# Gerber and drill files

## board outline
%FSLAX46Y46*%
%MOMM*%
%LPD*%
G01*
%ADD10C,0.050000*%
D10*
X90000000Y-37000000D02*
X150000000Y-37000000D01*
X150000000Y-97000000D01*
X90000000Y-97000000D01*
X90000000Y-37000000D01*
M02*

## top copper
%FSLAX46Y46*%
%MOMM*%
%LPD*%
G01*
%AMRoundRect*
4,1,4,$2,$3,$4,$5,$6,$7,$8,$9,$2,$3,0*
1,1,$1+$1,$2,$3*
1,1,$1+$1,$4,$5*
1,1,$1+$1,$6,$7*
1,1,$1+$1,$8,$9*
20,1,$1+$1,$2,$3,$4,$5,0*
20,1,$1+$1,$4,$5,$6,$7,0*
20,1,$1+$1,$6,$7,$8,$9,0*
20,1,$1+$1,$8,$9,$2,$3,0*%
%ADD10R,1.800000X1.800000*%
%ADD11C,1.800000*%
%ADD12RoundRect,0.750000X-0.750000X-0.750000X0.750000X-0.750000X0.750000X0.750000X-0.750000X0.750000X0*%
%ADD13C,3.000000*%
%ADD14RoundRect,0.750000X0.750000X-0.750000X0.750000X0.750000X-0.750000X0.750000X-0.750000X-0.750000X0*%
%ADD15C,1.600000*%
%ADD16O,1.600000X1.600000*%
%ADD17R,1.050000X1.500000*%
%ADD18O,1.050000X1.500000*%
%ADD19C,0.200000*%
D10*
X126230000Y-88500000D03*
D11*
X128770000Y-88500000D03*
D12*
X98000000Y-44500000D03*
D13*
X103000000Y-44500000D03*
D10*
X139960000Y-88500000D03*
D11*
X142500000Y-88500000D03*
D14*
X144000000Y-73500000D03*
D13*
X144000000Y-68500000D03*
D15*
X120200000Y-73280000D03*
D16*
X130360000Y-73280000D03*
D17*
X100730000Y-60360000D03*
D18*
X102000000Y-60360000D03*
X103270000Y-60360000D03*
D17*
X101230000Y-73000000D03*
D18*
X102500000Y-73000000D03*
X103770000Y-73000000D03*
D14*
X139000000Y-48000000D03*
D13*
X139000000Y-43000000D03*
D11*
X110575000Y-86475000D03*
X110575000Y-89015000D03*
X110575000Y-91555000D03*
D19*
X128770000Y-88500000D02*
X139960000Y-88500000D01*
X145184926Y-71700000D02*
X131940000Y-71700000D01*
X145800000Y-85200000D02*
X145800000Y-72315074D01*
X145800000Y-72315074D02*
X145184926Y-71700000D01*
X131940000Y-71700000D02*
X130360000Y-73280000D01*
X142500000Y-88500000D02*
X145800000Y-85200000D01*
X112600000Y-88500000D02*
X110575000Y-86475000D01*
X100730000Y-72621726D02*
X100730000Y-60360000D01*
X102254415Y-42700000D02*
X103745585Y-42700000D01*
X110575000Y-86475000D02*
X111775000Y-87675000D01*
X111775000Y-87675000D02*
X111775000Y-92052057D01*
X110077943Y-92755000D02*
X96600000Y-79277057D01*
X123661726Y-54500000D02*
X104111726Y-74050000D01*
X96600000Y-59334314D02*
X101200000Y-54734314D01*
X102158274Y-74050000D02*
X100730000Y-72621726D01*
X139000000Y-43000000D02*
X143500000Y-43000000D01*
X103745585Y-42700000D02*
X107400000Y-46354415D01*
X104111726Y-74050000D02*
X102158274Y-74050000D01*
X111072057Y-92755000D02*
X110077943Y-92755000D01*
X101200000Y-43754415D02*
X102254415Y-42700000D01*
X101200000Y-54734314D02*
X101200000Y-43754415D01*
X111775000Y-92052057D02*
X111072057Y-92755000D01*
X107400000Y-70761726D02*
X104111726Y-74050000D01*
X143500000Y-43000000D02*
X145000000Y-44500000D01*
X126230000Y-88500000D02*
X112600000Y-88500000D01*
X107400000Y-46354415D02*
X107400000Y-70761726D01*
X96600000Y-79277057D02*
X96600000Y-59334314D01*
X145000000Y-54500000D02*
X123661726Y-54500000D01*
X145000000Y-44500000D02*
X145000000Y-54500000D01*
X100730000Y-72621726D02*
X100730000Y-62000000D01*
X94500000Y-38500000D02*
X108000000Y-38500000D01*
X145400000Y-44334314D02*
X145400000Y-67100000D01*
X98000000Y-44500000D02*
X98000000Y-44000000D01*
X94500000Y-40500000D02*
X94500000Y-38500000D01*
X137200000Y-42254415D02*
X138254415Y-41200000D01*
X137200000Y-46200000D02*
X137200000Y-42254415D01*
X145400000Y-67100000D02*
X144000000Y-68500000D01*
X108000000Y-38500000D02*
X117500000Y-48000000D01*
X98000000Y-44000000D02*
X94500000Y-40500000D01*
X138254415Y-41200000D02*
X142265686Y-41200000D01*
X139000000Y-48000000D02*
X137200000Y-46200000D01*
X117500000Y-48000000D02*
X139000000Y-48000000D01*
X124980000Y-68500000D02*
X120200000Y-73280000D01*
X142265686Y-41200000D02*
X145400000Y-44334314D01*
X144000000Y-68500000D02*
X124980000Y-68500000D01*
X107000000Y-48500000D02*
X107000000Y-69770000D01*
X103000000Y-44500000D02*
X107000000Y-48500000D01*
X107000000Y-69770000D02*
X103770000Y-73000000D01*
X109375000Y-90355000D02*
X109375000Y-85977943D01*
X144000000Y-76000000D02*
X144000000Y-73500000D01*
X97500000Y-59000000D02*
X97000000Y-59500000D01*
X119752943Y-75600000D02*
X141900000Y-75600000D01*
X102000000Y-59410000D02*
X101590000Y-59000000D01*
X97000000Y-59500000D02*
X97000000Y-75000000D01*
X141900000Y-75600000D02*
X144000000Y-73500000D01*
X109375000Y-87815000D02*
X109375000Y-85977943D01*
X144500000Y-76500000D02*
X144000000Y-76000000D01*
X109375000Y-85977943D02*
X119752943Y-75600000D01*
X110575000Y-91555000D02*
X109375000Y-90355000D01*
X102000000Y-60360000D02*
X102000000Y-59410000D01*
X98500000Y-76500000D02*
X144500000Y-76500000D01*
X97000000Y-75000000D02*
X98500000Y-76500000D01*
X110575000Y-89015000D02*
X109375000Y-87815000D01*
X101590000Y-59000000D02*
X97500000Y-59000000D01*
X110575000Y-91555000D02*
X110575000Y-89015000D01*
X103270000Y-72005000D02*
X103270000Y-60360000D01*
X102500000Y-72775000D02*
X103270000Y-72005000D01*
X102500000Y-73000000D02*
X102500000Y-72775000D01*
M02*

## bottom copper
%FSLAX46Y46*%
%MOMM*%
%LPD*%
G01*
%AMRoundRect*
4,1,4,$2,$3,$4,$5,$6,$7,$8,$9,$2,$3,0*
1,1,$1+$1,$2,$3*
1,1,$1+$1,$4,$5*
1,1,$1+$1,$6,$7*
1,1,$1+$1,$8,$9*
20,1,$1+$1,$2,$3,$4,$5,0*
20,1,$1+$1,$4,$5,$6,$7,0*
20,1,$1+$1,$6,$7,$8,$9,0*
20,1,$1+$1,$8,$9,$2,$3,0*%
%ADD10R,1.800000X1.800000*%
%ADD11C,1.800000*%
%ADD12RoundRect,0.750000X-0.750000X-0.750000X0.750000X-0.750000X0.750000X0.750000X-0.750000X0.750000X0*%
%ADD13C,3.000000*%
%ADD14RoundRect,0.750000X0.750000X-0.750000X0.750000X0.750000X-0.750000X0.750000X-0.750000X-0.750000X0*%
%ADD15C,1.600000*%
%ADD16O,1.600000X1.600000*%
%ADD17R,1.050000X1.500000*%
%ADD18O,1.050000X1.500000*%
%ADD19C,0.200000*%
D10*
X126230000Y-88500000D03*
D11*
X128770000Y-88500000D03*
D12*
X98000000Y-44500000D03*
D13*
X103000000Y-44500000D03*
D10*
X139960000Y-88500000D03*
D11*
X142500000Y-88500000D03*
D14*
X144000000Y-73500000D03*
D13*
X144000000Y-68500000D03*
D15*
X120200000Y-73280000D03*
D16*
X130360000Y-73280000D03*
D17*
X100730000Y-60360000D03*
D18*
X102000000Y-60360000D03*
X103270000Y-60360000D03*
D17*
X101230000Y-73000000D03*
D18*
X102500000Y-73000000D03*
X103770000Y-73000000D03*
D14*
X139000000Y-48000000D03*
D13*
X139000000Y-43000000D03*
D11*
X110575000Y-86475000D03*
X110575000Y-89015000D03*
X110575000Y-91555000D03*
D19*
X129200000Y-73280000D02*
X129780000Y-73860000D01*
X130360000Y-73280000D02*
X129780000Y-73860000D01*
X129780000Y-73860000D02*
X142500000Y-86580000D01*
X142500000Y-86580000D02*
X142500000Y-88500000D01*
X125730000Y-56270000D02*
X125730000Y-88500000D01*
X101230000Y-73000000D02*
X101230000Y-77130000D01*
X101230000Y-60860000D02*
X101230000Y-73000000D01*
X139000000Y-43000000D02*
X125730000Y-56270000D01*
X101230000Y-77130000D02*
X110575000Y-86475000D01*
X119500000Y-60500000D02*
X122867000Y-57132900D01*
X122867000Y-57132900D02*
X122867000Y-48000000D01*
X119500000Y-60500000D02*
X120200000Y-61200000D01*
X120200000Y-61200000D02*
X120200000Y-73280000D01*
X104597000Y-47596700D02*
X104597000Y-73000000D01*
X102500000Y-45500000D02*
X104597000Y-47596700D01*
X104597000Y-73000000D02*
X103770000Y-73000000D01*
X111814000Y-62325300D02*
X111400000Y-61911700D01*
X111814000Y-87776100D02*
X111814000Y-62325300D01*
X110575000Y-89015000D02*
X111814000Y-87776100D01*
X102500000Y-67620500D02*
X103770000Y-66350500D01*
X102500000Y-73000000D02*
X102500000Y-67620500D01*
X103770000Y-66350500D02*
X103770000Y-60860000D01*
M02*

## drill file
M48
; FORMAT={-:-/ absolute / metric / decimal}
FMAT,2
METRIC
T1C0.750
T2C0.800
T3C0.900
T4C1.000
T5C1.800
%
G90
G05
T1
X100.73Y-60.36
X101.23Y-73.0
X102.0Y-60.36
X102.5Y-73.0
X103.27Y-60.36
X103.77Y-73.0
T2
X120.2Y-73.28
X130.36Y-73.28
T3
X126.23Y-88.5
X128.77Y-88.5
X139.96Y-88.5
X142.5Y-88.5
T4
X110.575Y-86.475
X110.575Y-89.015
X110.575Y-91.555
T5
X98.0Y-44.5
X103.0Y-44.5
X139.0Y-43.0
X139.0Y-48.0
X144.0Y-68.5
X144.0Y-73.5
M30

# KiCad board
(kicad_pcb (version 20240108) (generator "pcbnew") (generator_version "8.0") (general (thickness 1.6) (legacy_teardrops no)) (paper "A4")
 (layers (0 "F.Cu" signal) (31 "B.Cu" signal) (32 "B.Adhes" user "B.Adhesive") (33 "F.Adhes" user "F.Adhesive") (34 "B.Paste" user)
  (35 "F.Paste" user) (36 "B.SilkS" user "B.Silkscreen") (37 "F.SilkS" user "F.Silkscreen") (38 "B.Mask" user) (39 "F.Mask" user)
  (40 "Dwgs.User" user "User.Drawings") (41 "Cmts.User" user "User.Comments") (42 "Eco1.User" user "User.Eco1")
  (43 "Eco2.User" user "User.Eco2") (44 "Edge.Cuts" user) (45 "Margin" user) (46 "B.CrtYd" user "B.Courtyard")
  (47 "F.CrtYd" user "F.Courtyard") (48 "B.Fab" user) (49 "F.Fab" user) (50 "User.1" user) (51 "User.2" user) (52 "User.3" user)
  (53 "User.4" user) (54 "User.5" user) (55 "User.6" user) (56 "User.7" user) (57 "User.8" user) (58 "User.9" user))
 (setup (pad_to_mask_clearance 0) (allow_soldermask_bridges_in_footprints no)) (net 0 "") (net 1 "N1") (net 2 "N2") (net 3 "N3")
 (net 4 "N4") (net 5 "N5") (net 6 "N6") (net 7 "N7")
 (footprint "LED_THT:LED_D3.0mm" (layer "F.Cu") (at 126.23 88.5)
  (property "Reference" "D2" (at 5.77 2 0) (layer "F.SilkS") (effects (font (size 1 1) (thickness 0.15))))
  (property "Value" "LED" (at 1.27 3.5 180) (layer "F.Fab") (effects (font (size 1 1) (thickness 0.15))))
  (pad "1" thru_hole rect (at 0 0) (size 1.8 1.8) (drill 0.9) (layers "*.Cu" "*.Mask") (remove_unused_layers no) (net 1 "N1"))
  (pad "2" thru_hole circle (at 2.54 0) (size 1.8 1.8) (drill 0.9) (layers "*.Cu" "*.Mask") (remove_unused_layers no) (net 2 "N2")))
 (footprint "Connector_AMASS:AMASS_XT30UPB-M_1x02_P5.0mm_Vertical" (layer "F.Cu") (at 98 44.5)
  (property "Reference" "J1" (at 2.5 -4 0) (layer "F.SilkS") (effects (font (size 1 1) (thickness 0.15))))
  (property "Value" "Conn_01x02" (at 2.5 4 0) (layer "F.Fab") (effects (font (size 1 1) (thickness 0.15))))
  (pad "1" thru_hole roundrect (at 0 0) (size 3 3) (drill 1.8) (layers "*.Cu" "*.Mask") (remove_unused_layers no) (roundrect_rratio 0.25)
   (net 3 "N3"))
  (pad "2" thru_hole circle (at 5 0) (size 3 3) (drill 1.8) (layers "*.Cu" "*.Mask") (remove_unused_layers no) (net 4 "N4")))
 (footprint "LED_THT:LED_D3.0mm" (layer "F.Cu") (at 139.96 88.5)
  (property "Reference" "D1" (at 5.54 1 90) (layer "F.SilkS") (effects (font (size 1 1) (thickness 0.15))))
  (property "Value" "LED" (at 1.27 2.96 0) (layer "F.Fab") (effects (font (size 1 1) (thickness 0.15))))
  (pad "1" thru_hole rect (at 0 0) (size 1.8 1.8) (drill 0.9) (layers "*.Cu" "*.Mask") (remove_unused_layers no) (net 2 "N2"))
  (pad "2" thru_hole circle (at 2.54 0) (size 1.8 1.8) (drill 0.9) (layers "*.Cu" "*.Mask") (remove_unused_layers no) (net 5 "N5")))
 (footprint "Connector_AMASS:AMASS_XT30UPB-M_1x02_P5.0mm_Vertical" (layer "F.Cu") (at 144 73.5 90)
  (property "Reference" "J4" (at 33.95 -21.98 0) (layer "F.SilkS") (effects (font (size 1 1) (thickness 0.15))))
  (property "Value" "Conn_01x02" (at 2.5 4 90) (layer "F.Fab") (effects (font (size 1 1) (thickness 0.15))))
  (pad "1" thru_hole roundrect (at 0 0 90) (size 3 3) (drill 1.8) (layers "*.Cu" "*.Mask") (remove_unused_layers no) (roundrect_rratio 0.25)
   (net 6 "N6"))
  (pad "2" thru_hole circle (at 5 0 90) (size 3 3) (drill 1.8) (layers "*.Cu" "*.Mask") (remove_unused_layers no) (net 3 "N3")))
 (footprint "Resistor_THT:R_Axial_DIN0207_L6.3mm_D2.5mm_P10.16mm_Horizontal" (layer "F.Cu") (at 120.2 73.28)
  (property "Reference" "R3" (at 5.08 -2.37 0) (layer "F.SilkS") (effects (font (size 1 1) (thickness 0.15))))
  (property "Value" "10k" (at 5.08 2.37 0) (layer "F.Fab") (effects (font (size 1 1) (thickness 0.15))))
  (pad "1" thru_hole circle (at 0 0) (size 1.6 1.6) (drill 0.8) (layers "*.Cu" "*.Mask") (remove_unused_layers no) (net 3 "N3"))
  (pad "2" thru_hole oval (at 10.16 0) (size 1.6 1.6) (drill 0.8) (layers "*.Cu" "*.Mask") (remove_unused_layers no) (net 5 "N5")))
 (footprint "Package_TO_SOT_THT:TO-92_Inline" (layer "F.Cu") (at 100.73 60.36)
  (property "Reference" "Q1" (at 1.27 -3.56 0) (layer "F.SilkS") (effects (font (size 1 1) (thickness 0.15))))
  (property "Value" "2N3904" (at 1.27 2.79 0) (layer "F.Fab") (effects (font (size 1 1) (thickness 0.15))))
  (pad "1" thru_hole rect (at 0 0) (size 1.05 1.5) (drill 0.75) (layers "*.Cu" "*.Mask") (remove_unused_layers no) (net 1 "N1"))
  (pad "2" thru_hole oval (at 1.27 0) (size 1.05 1.5) (drill 0.75) (layers "*.Cu" "*.Mask") (remove_unused_layers no) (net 6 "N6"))
  (pad "3" thru_hole oval (at 2.54 0) (size 1.05 1.5) (drill 0.75) (layers "*.Cu" "*.Mask") (remove_unused_layers no) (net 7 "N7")))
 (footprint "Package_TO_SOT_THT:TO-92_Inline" (layer "F.Cu") (at 101.23 73)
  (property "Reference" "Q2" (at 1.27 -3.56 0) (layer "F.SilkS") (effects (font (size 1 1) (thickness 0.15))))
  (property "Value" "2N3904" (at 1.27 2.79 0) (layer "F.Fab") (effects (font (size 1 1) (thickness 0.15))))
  (pad "1" thru_hole rect (at 0 0) (size 1.05 1.5) (drill 0.75) (layers "*.Cu" "*.Mask") (remove_unused_layers no) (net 1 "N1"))
  (pad "2" thru_hole oval (at 1.27 0) (size 1.05 1.5) (drill 0.75) (layers "*.Cu" "*.Mask") (remove_unused_layers no) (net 7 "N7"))
  (pad "3" thru_hole oval (at 2.54 0) (size 1.05 1.5) (drill 0.75) (layers "*.Cu" "*.Mask") (remove_unused_layers no) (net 4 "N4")))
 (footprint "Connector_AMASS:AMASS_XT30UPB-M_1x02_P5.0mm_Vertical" (layer "F.Cu") (at 139 48 90)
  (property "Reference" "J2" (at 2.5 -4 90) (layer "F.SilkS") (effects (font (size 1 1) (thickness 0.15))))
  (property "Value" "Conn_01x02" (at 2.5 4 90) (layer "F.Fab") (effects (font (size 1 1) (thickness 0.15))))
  (pad "1" thru_hole roundrect (at 0 0 90) (size 3 3) (drill 1.8) (layers "*.Cu" "*.Mask") (remove_unused_layers no) (roundrect_rratio 0.25)
   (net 3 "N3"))
  (pad "2" thru_hole circle (at 5 0 90) (size 3 3) (drill 1.8) (layers "*.Cu" "*.Mask") (remove_unused_layers no) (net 1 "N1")))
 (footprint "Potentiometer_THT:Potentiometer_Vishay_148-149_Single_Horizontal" (layer "F.Cu") (at 110.575 86.475 180)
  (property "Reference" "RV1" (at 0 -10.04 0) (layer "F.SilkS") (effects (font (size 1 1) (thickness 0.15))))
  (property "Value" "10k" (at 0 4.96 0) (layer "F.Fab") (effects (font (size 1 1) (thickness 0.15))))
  (pad "1" thru_hole circle (at 0 0 180) (size 1.8 1.8) (drill 1) (layers "*.Cu" "*.Mask") (remove_unused_layers no) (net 1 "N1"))
  (pad "2" thru_hole circle (at 0 -2.54 180) (size 1.8 1.8) (drill 1) (layers "*.Cu" "*.Mask") (remove_unused_layers no) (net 6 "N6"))
  (pad "3" thru_hole circle (at 0 -5.08 180) (size 1.8 1.8) (drill 1) (layers "*.Cu" "*.Mask") (remove_unused_layers no) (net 6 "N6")))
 (gr_rect (start 90 37) (end 150 97) (stroke (width 0.05) (type default)) (fill none) (layer "Edge.Cuts"))
 (segment (start 128.77 88.5) (end 139.96 88.5) (width 0.2) (layer "F.Cu") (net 2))
 (segment (start 145.184926 71.7) (end 131.94 71.7) (width 0.2) (layer "F.Cu") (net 5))
 (segment (start 145.8 85.2) (end 145.8 72.315074) (width 0.2) (layer "F.Cu") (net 5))
 (segment (start 145.8 72.315074) (end 145.184926 71.7) (width 0.2) (layer "F.Cu") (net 5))
 (segment (start 131.94 71.7) (end 130.36 73.28) (width 0.2) (layer "F.Cu") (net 5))
 (segment (start 142.5 88.5) (end 145.8 85.2) (width 0.2) (layer "F.Cu") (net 5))
 (segment (start 129.2 73.28) (end 129.78 73.86) (width 0.2) (layer "B.Cu") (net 5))
 (segment (start 130.36 73.28) (end 129.78 73.86) (width 0.2) (layer "B.Cu") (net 5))
 (segment (start 129.78 73.86) (end 142.5 86.58) (width 0.2) (layer "B.Cu") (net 5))
 (segment (start 142.5 86.58) (end 142.5 88.5) (width 0.2) (layer "B.Cu") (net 5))
 (segment (start 112.6 88.5) (end 110.575 86.475) (width 0.2) (layer "F.Cu") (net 1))
 (segment (start 100.73 72.621726) (end 100.73 60.36) (width 0.2) (layer "F.Cu") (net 1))
 (segment (start 102.254415 42.7) (end 103.745585 42.7) (width 0.2) (layer "F.Cu") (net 1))
 (segment (start 110.575 86.475) (end 111.775 87.675) (width 0.2) (layer "F.Cu") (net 1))
 (segment (start 111.775 87.675) (end 111.775 92.052057) (width 0.2) (layer "F.Cu") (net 1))
 (segment (start 110.077943 92.755) (end 96.6 79.277057) (width 0.2) (layer "F.Cu") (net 1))
 (segment (start 123.661726 54.5) (end 104.111726 74.05) (width 0.2) (layer "F.Cu") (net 1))
 (segment (start 96.6 59.334314) (end 101.2 54.734314) (width 0.2) (layer "F.Cu") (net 1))
 (segment (start 102.158274 74.05) (end 100.73 72.621726) (width 0.2) (layer "F.Cu") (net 1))
 (segment (start 139 43) (end 143.5 43) (width 0.2) (layer "F.Cu") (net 1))
 (segment (start 103.745585 42.7) (end 107.4 46.354415) (width 0.2) (layer "F.Cu") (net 1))
 (segment (start 104.111726 74.05) (end 102.158274 74.05) (width 0.2) (layer "F.Cu") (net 1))
 (segment (start 111.072057 92.755) (end 110.077943 92.755) (width 0.2) (layer "F.Cu") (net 1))
 (segment (start 101.2 43.754415) (end 102.254415 42.7) (width 0.2) (layer "F.Cu") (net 1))
 (segment (start 101.2 54.734314) (end 101.2 43.754415) (width 0.2) (layer "F.Cu") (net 1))
 (segment (start 111.775 92.052057) (end 111.072057 92.755) (width 0.2) (layer "F.Cu") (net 1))
 (segment (start 107.4 70.761726) (end 104.111726 74.05) (width 0.2) (layer "F.Cu") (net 1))
 (segment (start 143.5 43) (end 145 44.5) (width 0.2) (layer "F.Cu") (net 1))
 (segment (start 126.23 88.5) (end 112.6 88.5) (width 0.2) (layer "F.Cu") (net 1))
 (segment (start 107.4 46.354415) (end 107.4 70.761726) (width 0.2) (layer "F.Cu") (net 1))
 (segment (start 96.6 79.277057) (end 96.6 59.334314) (width 0.2) (layer "F.Cu") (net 1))
 (segment (start 145 54.5) (end 123.661726 54.5) (width 0.2) (layer "F.Cu") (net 1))
 (segment (start 145 44.5) (end 145 54.5) (width 0.2) (layer "F.Cu") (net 1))
 (segment (start 100.73 72.621726) (end 100.73 62) (width 0.2) (layer "F.Cu") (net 1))
 (segment (start 125.73 56.27) (end 125.73 88.5) (width 0.2) (layer "B.Cu") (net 1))
 (segment (start 101.23 73) (end 101.23 77.13) (width 0.2) (layer "B.Cu") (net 1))
 (segment (start 101.23 60.86) (end 101.23 73) (width 0.2) (layer "B.Cu") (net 1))
 (segment (start 139 43) (end 125.73 56.27) (width 0.2) (layer "B.Cu") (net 1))
 (segment (start 101.23 77.13) (end 110.575 86.475) (width 0.2) (layer "B.Cu") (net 1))
 (segment (start 94.5 38.5) (end 108 38.5) (width 0.2) (layer "F.Cu") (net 3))
 (segment (start 145.4 44.334314) (end 145.4 67.1) (width 0.2) (layer "F.Cu") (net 3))
 (segment (start 98 44.5) (end 98 44) (width 0.2) (layer "F.Cu") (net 3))
 (segment (start 94.5 40.5) (end 94.5 38.5) (width 0.2) (layer "F.Cu") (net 3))
 (segment (start 137.2 42.254415) (end 138.254415 41.2) (width 0.2) (layer "F.Cu") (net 3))
 (segment (start 137.2 46.2) (end 137.2 42.254415) (width 0.2) (layer "F.Cu") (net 3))
 (segment (start 145.4 67.1) (end 144 68.5) (width 0.2) (layer "F.Cu") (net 3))
 (segment (start 108 38.5) (end 117.5 48) (width 0.2) (layer "F.Cu") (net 3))
 (segment (start 98 44) (end 94.5 40.5) (width 0.2) (layer "F.Cu") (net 3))
 (segment (start 138.254415 41.2) (end 142.265686 41.2) (width 0.2) (layer "F.Cu") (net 3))
 (segment (start 139 48) (end 137.2 46.2) (width 0.2) (layer "F.Cu") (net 3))
 (segment (start 117.5 48) (end 139 48) (width 0.2) (layer "F.Cu") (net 3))
 (segment (start 124.98 68.5) (end 120.2 73.28) (width 0.2) (layer "F.Cu") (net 3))
 (segment (start 142.265686 41.2) (end 145.4 44.334314) (width 0.2) (layer "F.Cu") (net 3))
 (segment (start 144 68.5) (end 124.98 68.5) (width 0.2) (layer "F.Cu") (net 3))
 (segment (start 119.5 60.5) (end 122.867 57.1329) (width 0.2) (layer "B.Cu") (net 3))
 (segment (start 122.867 57.1329) (end 122.867 48) (width 0.2) (layer "B.Cu") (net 3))
 (segment (start 119.5 60.5) (end 120.2 61.2) (width 0.2) (layer "B.Cu") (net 3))
 (segment (start 120.2 61.2) (end 120.2 73.28) (width 0.2) (layer "B.Cu") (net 3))
 (segment (start 107 48.5) (end 107 69.77) (width 0.2) (layer "F.Cu") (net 4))
 (segment (start 103 44.5) (end 107 48.5) (width 0.2) (layer "F.Cu") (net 4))
 (segment (start 107 69.77) (end 103.77 73) (width 0.2) (layer "F.Cu") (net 4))
 (segment (start 104.597 47.5967) (end 104.597 73) (width 0.2) (layer "B.Cu") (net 4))
 (segment (start 102.5 45.5) (end 104.597 47.5967) (width 0.2) (layer "B.Cu") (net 4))
 (segment (start 104.597 73) (end 103.77 73) (width 0.2) (layer "B.Cu") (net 4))
 (segment (start 109.375 90.355) (end 109.375 85.977943) (width 0.2) (layer "F.Cu") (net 6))
 (segment (start 144 76) (end 144 73.5) (width 0.2) (layer "F.Cu") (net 6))
 (segment (start 97.5 59) (end 97 59.5) (width 0.2) (layer "F.Cu") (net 6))
 (segment (start 119.752943 75.6) (end 141.9 75.6) (width 0.2) (layer "F.Cu") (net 6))
 (segment (start 102 59.41) (end 101.59 59) (width 0.2) (layer "F.Cu") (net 6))
 (segment (start 97 59.5) (end 97 75) (width 0.2) (layer "F.Cu") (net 6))
 (segment (start 141.9 75.6) (end 144 73.5) (width 0.2) (layer "F.Cu") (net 6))
 (segment (start 109.375 87.815) (end 109.375 85.977943) (width 0.2) (layer "F.Cu") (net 6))
 (segment (start 144.5 76.5) (end 144 76) (width 0.2) (layer "F.Cu") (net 6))
 (segment (start 109.375 85.977943) (end 119.752943 75.6) (width 0.2) (layer "F.Cu") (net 6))
 (segment (start 110.575 91.555) (end 109.375 90.355) (width 0.2) (layer "F.Cu") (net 6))
 (segment (start 102 60.36) (end 102 59.41) (width 0.2) (layer "F.Cu") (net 6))
 (segment (start 98.5 76.5) (end 144.5 76.5) (width 0.2) (layer "F.Cu") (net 6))
 (segment (start 97 75) (end 98.5 76.5) (width 0.2) (layer "F.Cu") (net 6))
 (segment (start 110.575 89.015) (end 109.375 87.815) (width 0.2) (layer "F.Cu") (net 6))
 (segment (start 101.59 59) (end 97.5 59) (width 0.2) (layer "F.Cu") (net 6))
 (segment (start 110.575 91.555) (end 110.575 89.015) (width 0.2) (layer "F.Cu") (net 6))
 (segment (start 111.814 62.3253) (end 111.4 61.9117) (width 0.2) (layer "B.Cu") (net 6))
 (segment (start 111.814 87.7761) (end 111.814 62.3253) (width 0.2) (layer "B.Cu") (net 6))
 (segment (start 110.575 89.015) (end 111.814 87.7761) (width 0.2) (layer "B.Cu") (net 6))
 (segment (start 103.27 72.005) (end 103.27 60.36) (width 0.2) (layer "F.Cu") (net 7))
 (segment (start 102.5 72.775) (end 103.27 72.005) (width 0.2) (layer "F.Cu") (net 7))
 (segment (start 102.5 73) (end 102.5 72.775) (width 0.2) (layer "F.Cu") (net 7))
 (segment (start 102.5 67.6205) (end 103.77 66.3505) (width 0.2) (layer "B.Cu") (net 7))
 (segment (start 102.5 73) (end 102.5 67.6205) (width 0.2) (layer "B.Cu") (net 7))
 (segment (start 103.77 66.3505) (end 103.77 60.86) (width 0.2) (layer "B.Cu") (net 7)))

